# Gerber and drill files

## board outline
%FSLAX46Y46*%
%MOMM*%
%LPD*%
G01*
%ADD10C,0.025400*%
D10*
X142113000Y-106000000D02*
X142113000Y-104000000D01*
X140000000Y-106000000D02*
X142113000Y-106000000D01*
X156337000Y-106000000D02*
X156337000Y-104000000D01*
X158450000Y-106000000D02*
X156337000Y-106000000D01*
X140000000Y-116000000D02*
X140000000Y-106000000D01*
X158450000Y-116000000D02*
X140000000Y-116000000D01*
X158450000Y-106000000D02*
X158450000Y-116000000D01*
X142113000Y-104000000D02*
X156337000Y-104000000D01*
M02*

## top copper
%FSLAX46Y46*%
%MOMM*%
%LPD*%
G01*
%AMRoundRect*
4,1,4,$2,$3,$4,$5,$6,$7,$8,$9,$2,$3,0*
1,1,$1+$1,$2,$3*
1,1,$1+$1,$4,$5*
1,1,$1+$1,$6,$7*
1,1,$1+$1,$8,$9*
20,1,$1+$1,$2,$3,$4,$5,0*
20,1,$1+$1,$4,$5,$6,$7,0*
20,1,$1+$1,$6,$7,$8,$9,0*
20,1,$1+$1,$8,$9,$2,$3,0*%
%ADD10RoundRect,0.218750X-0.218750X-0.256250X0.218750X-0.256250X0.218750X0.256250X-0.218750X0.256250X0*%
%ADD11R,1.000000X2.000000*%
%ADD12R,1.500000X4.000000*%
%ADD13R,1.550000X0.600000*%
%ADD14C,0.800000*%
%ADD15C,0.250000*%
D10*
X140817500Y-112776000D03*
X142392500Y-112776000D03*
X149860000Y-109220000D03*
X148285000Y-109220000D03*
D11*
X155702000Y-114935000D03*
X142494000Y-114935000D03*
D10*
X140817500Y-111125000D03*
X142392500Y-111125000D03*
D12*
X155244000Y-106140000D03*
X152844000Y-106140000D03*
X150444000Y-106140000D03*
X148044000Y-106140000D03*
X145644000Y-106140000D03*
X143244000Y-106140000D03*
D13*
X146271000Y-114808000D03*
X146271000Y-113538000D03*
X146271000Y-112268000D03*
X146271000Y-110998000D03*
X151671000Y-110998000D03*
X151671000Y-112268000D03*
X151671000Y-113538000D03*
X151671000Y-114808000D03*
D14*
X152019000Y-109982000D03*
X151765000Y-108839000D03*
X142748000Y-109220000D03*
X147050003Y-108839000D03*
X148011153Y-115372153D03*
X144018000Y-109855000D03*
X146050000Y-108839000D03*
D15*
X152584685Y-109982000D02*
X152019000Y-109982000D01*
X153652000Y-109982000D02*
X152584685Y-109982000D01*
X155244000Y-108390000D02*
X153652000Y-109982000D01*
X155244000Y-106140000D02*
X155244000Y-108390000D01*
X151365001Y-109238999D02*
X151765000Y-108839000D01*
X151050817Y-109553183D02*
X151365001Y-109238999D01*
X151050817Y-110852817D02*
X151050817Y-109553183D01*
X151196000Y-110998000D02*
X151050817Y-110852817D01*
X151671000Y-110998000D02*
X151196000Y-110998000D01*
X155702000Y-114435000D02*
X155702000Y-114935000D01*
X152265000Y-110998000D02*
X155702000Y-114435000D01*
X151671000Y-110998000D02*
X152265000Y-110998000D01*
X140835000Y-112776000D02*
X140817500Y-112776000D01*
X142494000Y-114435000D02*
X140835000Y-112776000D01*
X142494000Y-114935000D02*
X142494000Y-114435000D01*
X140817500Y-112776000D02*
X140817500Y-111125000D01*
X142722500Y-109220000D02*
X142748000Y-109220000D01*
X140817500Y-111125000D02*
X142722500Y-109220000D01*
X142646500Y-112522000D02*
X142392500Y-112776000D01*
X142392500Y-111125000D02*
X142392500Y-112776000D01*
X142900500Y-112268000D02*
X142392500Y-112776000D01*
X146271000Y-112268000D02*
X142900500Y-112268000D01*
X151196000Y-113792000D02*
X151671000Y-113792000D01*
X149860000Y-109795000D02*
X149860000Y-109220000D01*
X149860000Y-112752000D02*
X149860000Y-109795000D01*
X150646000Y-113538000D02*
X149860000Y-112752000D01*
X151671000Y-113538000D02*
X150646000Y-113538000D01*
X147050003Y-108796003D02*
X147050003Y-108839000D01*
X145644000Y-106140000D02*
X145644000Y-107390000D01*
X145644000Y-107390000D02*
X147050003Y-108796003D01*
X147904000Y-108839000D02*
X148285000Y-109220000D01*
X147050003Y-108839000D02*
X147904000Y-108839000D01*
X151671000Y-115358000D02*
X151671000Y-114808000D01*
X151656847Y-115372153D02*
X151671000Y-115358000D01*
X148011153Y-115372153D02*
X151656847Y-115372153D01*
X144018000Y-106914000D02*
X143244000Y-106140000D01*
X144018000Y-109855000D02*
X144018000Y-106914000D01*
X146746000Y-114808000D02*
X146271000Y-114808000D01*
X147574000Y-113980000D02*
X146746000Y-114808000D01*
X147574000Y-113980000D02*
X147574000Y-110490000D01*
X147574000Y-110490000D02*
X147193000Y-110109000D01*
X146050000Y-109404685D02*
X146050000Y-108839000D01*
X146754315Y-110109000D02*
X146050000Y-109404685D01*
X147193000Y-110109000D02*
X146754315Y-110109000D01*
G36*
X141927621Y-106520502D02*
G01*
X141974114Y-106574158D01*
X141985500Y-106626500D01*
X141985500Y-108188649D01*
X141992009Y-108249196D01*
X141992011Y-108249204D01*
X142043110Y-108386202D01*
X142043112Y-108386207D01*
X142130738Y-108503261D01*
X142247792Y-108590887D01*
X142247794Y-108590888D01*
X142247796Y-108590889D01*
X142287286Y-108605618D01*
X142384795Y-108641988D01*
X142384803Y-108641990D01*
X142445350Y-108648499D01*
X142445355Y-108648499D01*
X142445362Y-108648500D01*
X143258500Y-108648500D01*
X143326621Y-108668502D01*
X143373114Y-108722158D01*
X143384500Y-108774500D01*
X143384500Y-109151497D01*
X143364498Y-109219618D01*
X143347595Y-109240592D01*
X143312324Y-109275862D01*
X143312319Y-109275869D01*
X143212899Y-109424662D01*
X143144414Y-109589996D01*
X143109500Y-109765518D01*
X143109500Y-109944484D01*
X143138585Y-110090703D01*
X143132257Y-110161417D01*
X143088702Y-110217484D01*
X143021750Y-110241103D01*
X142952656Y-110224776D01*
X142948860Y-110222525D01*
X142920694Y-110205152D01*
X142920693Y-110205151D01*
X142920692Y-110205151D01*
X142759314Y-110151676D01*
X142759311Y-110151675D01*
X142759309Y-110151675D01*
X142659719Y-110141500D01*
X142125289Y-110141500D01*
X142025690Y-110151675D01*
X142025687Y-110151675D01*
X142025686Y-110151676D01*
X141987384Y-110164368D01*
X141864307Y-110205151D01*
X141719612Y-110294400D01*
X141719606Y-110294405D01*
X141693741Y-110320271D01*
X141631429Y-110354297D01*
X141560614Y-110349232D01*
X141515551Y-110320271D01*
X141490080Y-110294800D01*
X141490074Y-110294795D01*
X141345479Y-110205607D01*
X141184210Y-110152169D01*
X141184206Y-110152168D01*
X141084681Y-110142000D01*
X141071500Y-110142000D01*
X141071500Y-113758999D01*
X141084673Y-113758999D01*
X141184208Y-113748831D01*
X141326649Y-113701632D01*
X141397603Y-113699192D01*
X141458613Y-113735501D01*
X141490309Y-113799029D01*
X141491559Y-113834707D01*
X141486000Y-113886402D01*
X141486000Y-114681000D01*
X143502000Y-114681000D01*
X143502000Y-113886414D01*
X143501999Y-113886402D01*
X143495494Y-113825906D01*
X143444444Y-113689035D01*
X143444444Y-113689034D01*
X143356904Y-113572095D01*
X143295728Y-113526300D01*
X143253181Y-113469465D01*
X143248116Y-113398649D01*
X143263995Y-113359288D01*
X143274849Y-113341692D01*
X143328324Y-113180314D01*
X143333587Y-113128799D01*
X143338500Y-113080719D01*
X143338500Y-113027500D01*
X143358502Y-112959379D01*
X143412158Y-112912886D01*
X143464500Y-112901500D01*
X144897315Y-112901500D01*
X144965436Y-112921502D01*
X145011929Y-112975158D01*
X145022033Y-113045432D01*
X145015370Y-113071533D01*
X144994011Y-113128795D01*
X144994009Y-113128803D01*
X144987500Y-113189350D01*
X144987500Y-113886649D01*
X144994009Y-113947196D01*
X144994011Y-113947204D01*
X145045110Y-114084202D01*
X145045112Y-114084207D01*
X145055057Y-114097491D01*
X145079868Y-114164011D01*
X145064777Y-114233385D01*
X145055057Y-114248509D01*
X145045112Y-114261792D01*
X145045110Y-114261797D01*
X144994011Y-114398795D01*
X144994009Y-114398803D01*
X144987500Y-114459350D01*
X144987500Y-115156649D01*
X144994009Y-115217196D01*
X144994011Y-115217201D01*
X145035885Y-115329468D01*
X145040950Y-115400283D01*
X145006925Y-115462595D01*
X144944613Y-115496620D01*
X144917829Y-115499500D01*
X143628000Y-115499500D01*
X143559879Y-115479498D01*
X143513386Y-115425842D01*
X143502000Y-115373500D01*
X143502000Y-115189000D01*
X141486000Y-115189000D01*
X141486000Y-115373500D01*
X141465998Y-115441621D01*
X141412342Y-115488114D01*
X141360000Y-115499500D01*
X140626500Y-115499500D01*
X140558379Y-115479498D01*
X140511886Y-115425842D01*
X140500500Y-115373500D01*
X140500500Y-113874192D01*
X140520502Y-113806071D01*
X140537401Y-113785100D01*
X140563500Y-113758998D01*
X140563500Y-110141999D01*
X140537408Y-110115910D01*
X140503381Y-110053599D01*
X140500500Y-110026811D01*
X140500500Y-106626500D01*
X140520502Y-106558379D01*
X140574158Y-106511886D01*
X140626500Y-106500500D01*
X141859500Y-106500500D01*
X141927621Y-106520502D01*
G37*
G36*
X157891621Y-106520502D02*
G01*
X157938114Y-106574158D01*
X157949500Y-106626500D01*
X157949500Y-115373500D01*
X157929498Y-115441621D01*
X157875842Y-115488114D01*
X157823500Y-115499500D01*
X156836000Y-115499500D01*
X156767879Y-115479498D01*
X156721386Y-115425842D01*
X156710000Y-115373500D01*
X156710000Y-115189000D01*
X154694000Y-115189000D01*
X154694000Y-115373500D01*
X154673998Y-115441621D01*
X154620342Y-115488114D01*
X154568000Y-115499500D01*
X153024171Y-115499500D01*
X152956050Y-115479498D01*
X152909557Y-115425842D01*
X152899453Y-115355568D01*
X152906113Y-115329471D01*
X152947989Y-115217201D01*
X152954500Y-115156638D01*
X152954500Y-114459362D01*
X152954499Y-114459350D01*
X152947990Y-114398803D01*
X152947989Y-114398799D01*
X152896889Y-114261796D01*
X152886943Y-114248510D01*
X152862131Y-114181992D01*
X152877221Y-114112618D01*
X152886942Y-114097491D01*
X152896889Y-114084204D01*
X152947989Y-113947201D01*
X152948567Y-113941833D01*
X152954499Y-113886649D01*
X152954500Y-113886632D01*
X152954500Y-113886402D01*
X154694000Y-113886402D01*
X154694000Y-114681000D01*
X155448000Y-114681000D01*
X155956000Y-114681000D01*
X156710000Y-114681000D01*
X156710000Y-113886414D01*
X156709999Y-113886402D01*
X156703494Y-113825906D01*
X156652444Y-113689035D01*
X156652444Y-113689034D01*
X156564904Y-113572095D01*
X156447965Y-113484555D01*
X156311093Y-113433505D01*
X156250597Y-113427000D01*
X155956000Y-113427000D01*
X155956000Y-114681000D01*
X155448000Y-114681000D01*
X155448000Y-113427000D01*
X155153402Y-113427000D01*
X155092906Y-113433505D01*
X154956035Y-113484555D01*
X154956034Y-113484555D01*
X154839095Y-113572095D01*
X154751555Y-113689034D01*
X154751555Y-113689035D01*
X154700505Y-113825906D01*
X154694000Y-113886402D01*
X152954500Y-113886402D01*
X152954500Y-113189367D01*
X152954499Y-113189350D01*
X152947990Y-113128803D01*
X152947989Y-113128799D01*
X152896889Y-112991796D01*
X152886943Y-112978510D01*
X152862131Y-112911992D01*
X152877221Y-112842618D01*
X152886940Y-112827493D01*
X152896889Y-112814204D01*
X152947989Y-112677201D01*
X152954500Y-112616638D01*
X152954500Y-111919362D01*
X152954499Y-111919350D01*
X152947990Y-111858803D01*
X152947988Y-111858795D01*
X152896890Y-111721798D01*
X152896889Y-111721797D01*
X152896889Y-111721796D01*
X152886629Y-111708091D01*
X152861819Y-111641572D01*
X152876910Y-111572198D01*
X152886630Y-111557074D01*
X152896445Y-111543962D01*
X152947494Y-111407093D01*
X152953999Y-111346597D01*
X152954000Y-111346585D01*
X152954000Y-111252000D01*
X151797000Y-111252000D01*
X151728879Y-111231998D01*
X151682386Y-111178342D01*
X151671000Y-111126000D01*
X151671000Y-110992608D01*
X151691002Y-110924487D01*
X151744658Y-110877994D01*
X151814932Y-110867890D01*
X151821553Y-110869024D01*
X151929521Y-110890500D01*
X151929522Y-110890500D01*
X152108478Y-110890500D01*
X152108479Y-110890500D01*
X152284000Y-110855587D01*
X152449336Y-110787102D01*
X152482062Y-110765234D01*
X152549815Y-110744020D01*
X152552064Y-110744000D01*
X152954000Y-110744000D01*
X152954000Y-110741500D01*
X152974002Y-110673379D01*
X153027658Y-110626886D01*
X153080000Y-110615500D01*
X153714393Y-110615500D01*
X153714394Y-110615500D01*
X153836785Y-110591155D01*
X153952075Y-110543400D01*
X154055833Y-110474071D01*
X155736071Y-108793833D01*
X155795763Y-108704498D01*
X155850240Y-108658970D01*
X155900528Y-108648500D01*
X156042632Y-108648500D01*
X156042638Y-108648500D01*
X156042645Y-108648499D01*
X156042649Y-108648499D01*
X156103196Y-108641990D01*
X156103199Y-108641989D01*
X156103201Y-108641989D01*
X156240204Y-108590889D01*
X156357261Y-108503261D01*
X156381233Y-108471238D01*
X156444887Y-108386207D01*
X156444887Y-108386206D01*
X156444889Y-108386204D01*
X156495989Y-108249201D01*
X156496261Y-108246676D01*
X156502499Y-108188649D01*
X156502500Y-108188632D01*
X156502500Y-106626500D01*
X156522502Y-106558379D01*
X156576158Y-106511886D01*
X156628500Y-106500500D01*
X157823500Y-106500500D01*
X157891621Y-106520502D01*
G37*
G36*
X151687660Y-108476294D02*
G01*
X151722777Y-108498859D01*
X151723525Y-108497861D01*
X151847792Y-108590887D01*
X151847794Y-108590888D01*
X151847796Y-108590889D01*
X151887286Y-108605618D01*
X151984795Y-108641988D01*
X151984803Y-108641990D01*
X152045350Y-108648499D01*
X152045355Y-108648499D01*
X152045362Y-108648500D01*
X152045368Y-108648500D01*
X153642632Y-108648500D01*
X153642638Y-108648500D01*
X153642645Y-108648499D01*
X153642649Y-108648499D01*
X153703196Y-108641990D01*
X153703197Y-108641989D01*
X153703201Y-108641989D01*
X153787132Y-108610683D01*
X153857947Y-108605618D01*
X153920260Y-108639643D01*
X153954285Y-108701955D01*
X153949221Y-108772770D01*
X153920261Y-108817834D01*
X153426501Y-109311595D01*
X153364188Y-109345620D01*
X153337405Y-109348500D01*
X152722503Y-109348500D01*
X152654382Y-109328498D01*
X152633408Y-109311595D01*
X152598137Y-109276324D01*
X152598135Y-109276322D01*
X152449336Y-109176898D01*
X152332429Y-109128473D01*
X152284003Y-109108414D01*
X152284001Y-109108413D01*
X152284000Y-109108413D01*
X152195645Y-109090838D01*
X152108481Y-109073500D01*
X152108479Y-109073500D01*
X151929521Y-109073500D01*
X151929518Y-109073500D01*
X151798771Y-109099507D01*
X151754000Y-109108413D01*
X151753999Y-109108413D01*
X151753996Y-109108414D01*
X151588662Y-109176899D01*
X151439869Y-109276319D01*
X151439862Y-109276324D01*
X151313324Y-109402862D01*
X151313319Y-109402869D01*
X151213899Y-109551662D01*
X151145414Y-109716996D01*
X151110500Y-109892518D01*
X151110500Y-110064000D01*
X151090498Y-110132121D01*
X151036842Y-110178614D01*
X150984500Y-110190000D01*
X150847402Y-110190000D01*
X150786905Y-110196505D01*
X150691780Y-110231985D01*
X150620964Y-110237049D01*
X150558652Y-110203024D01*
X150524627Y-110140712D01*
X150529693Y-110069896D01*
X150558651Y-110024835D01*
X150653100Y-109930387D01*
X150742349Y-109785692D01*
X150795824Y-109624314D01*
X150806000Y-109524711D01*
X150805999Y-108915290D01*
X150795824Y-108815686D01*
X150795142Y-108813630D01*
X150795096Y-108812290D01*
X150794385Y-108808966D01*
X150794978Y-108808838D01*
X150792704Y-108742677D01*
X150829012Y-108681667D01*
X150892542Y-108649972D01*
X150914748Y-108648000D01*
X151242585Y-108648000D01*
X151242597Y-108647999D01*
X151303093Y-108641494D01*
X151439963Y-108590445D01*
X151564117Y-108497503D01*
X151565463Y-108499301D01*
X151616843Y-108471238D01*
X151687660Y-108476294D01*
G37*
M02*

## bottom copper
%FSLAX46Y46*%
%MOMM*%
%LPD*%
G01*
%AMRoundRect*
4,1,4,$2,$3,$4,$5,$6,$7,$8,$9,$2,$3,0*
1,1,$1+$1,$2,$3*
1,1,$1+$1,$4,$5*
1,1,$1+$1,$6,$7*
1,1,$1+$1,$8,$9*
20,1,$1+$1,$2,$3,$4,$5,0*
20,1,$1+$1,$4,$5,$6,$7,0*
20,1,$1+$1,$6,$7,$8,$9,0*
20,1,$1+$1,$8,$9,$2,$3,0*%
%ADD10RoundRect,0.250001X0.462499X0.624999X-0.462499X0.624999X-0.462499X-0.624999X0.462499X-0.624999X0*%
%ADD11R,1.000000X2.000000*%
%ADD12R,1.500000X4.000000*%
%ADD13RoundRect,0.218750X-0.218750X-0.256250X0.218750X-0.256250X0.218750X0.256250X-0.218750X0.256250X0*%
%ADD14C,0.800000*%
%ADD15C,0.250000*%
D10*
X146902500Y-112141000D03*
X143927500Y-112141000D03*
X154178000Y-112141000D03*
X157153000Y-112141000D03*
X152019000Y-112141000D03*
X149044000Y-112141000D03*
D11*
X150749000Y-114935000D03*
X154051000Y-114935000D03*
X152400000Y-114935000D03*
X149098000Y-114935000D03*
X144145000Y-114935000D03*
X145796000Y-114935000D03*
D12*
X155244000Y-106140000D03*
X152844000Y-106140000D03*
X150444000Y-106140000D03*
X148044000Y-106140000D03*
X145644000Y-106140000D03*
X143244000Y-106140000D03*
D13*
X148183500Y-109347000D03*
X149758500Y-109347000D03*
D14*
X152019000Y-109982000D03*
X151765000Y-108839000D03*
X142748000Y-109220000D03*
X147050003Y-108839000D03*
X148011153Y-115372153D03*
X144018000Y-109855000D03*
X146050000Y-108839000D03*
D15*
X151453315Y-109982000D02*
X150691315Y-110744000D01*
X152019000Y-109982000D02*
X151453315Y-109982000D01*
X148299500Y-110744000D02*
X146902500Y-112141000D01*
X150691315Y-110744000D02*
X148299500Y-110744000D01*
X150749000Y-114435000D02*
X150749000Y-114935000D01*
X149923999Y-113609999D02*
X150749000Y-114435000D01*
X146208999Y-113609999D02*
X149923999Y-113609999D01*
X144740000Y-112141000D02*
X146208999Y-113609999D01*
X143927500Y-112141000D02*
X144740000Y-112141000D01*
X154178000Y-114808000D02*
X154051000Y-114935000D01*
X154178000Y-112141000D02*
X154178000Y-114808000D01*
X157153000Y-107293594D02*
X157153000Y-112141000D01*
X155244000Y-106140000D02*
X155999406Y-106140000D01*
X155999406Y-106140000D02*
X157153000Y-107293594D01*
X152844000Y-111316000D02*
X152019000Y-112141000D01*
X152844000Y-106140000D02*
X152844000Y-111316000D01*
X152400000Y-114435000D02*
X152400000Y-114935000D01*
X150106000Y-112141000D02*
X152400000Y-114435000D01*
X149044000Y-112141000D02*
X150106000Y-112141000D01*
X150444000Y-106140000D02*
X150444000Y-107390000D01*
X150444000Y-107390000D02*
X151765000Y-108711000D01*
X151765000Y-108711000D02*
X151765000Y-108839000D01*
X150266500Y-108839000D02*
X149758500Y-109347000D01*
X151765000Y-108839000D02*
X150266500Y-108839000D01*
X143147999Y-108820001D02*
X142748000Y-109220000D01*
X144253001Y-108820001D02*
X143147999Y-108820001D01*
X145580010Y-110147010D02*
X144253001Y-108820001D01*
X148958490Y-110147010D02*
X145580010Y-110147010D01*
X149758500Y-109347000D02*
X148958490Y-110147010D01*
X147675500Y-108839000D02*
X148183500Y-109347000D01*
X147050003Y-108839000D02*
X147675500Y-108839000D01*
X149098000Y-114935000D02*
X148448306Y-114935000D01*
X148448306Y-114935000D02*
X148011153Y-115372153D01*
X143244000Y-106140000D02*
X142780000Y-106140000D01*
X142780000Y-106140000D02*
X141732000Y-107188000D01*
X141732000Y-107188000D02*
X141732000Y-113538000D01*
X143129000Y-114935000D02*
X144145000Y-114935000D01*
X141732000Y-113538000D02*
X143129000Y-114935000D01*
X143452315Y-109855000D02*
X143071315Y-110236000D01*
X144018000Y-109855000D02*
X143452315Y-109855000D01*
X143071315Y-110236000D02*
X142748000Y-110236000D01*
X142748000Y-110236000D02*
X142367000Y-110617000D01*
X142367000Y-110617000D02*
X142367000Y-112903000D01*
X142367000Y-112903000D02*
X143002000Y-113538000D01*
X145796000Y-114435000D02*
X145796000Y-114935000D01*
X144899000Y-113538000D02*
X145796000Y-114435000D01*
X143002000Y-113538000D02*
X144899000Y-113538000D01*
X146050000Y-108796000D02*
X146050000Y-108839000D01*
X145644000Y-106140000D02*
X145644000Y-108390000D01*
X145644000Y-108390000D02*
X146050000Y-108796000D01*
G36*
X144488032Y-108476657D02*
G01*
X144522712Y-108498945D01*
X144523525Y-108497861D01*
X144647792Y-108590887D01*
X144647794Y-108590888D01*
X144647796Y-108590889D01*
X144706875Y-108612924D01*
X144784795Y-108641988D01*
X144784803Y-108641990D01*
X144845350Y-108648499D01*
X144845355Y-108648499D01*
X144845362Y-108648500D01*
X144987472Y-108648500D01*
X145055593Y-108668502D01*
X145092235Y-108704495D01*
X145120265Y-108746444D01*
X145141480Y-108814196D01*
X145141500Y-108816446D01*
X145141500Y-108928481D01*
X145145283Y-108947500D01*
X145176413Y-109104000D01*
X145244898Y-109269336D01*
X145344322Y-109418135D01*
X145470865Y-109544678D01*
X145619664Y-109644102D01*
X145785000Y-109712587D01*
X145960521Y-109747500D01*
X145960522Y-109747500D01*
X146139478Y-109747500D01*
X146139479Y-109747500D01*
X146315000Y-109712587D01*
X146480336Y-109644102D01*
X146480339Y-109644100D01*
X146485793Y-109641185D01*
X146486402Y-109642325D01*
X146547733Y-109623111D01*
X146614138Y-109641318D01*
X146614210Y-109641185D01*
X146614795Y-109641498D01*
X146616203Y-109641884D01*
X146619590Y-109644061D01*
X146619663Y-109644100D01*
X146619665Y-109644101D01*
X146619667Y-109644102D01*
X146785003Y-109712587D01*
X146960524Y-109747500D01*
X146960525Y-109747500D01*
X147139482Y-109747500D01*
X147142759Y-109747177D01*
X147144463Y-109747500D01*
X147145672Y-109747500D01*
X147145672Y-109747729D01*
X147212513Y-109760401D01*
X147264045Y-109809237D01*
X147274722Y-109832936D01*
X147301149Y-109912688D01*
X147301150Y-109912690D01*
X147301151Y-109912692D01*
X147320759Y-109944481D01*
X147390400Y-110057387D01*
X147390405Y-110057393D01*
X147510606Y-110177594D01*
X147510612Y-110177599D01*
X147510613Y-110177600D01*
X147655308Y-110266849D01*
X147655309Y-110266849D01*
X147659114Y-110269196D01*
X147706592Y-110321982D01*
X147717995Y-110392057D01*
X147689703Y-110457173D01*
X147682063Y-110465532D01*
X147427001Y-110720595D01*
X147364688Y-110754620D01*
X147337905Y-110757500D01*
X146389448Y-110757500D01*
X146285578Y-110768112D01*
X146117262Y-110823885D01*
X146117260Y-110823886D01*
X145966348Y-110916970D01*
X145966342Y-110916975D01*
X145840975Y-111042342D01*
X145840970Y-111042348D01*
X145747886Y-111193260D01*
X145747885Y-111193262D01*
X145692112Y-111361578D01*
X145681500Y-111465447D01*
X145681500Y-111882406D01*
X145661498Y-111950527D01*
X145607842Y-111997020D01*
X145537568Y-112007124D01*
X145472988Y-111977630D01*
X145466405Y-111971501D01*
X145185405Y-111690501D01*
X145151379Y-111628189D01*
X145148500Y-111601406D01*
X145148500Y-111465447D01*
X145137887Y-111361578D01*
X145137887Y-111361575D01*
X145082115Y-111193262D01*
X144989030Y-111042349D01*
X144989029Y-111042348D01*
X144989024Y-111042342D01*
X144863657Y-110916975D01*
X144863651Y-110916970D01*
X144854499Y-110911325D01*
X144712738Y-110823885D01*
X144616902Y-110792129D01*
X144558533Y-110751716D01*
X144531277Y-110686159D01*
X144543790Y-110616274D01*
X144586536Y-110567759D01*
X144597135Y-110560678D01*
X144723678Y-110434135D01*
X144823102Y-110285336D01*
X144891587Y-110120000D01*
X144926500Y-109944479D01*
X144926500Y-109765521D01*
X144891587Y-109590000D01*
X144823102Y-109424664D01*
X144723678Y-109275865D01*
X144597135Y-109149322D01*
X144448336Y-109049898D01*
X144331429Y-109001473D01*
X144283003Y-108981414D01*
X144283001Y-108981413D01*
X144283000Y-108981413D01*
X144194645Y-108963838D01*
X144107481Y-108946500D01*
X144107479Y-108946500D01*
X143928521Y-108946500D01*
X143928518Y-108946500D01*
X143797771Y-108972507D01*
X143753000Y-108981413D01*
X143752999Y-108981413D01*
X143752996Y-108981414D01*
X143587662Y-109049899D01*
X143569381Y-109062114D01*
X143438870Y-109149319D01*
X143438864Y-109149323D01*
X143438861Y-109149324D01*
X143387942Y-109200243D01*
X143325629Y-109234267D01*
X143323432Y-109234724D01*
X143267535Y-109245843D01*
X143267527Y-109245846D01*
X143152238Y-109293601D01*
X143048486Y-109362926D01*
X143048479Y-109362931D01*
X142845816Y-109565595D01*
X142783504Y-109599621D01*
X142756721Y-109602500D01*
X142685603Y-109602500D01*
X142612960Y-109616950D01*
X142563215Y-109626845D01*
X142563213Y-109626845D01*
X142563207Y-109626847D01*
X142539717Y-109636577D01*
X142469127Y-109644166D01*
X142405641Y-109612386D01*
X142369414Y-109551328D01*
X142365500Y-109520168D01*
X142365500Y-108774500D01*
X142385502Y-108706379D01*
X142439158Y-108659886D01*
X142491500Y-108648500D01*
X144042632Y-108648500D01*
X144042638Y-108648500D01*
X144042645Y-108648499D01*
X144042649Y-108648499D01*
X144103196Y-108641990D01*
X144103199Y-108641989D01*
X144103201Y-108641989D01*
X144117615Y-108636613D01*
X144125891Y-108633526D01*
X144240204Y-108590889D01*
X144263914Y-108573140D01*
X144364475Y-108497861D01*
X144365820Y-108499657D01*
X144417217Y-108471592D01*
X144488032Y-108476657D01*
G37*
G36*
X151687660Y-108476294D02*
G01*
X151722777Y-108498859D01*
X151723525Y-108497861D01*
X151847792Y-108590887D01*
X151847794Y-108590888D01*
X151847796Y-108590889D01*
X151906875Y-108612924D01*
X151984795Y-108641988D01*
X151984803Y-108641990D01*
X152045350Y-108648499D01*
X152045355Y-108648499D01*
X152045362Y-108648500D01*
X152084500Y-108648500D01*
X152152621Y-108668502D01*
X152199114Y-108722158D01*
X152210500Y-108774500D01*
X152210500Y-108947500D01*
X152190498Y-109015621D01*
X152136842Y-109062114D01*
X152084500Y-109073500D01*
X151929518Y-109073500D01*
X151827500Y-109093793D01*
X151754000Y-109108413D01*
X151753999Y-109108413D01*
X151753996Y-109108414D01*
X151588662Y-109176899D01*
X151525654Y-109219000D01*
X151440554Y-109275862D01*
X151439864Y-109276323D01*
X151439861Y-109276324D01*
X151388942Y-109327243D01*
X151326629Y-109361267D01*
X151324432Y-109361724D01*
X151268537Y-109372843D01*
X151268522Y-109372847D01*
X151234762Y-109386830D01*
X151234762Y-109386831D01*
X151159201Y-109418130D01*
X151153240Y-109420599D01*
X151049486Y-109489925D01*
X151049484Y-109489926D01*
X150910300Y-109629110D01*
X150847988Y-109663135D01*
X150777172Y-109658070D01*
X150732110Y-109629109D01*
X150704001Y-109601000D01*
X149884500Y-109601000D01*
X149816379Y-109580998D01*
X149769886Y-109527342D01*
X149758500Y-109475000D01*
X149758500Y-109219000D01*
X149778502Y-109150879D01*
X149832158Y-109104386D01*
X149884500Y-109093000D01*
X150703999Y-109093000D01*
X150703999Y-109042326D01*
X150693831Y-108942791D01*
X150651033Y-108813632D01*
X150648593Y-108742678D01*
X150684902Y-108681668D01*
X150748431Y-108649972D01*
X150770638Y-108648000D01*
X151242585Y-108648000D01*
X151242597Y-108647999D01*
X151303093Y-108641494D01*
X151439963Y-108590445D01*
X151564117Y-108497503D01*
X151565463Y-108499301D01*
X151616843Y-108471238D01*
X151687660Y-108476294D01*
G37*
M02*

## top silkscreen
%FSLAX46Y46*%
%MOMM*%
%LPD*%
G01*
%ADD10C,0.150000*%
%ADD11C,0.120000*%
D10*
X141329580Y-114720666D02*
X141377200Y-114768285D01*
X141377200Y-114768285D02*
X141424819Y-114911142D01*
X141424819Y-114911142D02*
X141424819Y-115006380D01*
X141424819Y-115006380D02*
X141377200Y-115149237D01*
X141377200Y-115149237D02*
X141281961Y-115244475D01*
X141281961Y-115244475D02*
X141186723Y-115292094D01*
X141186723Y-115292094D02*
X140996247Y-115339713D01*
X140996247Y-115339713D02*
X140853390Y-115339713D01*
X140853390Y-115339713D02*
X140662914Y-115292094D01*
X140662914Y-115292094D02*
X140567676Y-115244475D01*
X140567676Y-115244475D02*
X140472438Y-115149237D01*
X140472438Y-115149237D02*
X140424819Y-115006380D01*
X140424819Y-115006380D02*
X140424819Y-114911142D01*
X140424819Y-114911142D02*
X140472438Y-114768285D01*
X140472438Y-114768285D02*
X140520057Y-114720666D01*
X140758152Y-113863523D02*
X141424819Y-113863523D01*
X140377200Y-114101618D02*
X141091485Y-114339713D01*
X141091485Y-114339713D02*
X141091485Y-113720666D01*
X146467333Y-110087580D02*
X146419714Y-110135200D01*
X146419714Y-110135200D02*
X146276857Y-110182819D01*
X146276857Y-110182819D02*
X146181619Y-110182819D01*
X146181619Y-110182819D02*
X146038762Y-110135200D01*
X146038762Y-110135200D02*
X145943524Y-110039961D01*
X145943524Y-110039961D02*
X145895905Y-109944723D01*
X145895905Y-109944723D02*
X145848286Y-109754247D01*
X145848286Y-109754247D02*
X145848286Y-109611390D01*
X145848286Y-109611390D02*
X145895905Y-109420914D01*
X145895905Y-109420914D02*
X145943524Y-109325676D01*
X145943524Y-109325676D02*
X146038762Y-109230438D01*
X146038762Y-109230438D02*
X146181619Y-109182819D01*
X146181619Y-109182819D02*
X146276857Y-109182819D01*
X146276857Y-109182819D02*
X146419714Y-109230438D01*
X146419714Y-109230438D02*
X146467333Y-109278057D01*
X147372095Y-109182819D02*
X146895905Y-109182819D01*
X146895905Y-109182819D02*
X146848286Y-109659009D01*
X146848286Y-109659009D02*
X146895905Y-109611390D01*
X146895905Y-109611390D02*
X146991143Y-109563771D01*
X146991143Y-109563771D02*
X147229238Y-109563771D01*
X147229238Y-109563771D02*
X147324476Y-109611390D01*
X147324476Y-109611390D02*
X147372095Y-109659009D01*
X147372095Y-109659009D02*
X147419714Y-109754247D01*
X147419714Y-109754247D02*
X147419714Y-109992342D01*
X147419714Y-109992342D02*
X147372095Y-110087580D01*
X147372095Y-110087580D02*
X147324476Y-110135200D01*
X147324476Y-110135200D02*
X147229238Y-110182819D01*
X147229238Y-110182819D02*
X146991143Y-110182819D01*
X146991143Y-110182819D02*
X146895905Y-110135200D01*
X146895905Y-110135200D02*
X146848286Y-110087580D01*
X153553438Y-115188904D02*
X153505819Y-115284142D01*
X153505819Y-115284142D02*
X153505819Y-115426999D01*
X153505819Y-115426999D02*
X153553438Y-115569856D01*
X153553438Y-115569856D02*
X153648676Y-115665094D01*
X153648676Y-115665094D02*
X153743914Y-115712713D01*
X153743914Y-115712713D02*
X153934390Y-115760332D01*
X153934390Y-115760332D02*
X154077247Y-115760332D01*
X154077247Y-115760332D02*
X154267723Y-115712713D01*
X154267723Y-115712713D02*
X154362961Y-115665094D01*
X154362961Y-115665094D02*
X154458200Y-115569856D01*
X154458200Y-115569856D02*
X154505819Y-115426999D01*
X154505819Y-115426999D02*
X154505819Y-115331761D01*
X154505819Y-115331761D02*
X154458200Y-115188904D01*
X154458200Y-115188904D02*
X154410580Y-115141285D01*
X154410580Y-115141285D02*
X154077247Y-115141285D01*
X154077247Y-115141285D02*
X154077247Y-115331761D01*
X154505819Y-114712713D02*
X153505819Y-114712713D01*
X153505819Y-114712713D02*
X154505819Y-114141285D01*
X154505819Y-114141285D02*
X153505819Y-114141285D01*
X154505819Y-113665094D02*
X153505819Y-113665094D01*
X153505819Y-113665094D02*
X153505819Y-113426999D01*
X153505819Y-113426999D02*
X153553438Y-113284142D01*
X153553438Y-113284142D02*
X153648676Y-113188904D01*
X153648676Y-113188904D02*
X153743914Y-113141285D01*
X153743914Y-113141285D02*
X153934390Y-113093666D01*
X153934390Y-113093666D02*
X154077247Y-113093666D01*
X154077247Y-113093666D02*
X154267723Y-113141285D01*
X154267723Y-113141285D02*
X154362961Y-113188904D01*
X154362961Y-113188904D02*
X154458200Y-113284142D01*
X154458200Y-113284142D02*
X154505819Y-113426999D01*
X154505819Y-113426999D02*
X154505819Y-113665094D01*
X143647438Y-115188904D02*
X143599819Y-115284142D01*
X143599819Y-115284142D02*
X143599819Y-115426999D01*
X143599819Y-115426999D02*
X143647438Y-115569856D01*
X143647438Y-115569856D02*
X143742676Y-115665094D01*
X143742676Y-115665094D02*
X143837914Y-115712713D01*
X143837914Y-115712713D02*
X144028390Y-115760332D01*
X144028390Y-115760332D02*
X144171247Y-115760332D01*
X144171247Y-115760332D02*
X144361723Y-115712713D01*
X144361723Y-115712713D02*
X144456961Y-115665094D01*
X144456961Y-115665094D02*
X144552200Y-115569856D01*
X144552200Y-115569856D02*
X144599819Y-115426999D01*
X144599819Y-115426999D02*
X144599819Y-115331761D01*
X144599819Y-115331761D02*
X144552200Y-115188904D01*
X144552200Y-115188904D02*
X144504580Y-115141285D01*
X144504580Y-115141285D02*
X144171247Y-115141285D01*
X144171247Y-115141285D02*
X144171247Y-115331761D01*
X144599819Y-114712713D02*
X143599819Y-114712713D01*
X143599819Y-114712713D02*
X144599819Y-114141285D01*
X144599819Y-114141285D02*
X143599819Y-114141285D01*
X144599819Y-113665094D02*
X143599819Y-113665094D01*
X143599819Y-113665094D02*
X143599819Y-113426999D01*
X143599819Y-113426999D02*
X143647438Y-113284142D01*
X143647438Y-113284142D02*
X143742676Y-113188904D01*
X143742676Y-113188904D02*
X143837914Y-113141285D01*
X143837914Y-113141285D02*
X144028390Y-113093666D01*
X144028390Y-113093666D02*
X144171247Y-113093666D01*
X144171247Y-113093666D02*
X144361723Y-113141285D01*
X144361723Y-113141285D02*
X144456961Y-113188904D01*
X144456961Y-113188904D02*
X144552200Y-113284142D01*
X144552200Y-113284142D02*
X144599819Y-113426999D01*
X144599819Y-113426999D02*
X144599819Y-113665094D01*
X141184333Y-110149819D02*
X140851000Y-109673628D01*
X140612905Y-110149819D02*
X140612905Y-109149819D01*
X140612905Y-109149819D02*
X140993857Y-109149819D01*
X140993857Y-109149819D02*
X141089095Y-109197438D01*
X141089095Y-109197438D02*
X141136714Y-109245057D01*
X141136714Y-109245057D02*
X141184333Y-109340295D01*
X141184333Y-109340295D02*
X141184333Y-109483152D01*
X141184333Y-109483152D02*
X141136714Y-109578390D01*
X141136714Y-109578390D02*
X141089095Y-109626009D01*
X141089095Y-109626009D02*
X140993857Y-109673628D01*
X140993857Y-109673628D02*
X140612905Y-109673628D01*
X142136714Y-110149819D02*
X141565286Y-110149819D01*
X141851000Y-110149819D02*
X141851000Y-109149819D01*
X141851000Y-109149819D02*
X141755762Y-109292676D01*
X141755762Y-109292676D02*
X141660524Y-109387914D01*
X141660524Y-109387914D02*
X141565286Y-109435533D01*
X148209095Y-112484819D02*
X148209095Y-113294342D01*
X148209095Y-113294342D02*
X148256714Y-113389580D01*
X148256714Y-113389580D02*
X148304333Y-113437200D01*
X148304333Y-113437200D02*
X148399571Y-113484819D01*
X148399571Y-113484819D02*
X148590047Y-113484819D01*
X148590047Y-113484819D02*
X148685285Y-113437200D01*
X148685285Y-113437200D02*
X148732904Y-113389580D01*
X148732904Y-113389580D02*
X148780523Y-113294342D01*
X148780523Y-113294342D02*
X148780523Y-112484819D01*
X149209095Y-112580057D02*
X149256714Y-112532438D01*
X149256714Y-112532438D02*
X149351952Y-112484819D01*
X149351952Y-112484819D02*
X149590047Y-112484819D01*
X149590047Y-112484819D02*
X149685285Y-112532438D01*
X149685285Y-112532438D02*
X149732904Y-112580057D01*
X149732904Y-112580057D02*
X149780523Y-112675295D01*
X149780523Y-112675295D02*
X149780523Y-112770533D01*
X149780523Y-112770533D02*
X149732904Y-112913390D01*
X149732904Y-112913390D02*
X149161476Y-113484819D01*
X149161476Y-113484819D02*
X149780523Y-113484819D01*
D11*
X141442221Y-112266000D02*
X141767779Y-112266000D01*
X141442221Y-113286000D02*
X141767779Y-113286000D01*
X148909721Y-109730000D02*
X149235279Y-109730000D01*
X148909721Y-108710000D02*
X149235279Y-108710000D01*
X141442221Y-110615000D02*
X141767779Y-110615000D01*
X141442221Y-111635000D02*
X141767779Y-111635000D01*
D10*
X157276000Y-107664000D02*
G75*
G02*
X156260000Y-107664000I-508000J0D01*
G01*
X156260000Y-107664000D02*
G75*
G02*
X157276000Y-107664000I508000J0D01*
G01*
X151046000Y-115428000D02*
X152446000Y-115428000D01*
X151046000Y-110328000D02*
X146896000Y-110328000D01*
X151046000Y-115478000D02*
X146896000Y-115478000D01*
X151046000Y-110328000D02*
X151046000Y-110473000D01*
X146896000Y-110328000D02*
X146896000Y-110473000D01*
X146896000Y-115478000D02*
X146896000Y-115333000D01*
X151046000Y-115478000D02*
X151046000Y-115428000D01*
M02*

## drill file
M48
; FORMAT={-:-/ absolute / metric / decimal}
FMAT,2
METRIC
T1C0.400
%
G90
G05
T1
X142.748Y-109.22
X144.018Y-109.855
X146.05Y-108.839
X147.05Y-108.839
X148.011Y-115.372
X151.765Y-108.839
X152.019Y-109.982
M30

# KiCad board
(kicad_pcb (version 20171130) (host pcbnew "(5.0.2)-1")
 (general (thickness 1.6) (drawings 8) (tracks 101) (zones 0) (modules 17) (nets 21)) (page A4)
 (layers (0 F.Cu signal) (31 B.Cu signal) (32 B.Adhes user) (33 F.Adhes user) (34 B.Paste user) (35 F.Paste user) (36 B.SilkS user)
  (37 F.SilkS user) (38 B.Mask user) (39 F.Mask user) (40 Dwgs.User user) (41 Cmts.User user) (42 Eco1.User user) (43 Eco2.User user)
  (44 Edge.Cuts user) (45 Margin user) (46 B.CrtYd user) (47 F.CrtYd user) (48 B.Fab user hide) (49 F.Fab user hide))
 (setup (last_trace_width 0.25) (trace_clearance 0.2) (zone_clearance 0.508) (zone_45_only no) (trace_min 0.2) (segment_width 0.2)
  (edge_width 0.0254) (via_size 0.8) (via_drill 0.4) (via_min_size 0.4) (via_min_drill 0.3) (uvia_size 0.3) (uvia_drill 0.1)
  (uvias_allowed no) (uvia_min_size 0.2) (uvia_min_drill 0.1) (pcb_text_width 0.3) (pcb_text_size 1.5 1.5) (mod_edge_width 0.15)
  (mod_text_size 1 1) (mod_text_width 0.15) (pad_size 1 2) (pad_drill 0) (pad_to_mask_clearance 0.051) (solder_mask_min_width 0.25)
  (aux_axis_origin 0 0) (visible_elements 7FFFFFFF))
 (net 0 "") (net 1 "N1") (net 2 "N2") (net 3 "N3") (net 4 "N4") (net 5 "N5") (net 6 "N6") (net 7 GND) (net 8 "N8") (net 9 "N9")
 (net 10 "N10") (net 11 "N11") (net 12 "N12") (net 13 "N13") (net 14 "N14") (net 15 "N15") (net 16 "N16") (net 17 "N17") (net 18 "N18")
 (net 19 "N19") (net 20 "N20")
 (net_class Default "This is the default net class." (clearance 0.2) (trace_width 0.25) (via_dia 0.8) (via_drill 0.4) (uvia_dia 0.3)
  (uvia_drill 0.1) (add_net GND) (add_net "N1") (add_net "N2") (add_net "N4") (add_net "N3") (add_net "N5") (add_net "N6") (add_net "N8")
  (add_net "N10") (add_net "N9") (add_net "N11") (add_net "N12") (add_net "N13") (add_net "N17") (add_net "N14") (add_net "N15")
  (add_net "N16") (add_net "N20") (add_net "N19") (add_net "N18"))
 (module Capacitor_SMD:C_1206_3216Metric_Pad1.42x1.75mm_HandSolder (layer B.Cu) (at 145.415 112.141 180)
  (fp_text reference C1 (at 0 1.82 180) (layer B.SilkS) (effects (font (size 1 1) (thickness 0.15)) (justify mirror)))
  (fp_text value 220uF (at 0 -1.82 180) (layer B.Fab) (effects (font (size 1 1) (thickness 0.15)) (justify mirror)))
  (pad 1 smd roundrect (at -1.4875 0 180) (size 1.425 1.75) (layers B.Cu B.Paste B.Mask) (roundrect_rratio 0.175439) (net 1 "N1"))
  (pad 2 smd roundrect (at 1.4875 0 180) (size 1.425 1.75) (layers B.Cu B.Paste B.Mask) (roundrect_rratio 0.175439) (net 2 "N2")))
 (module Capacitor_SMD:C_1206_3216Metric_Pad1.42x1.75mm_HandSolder (layer B.Cu) (at 155.6655 112.141 180)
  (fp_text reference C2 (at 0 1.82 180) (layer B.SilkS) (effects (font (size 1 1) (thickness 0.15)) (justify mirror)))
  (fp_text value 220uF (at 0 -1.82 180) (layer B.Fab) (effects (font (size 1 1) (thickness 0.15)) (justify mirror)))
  (pad 2 smd roundrect (at 1.4875 0 180) (size 1.425 1.75) (layers B.Cu B.Paste B.Mask) (roundrect_rratio 0.175439) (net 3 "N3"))
  (pad 1 smd roundrect (at -1.4875 0 180) (size 1.425 1.75) (layers B.Cu B.Paste B.Mask) (roundrect_rratio 0.175439) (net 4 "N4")))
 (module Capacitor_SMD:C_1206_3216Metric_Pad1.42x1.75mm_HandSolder (layer B.Cu) (at 150.5315 112.141 180)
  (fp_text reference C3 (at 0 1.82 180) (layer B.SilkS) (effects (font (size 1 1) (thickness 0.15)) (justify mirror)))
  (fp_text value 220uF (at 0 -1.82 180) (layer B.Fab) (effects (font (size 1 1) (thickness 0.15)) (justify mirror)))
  (pad 1 smd roundrect (at -1.4875 0 180) (size 1.425 1.75) (layers B.Cu B.Paste B.Mask) (roundrect_rratio 0.175439) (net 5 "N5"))
  (pad 2 smd roundrect (at 1.4875 0 180) (size 1.425 1.75) (layers B.Cu B.Paste B.Mask) (roundrect_rratio 0.175439) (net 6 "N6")))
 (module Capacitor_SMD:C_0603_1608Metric (layer F.Cu) (at 141.605 112.776)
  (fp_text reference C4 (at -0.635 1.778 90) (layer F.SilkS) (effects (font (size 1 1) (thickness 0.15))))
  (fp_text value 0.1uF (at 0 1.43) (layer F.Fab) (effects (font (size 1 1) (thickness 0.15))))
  (fp_line (start -0.162779 -0.51) (end 0.162779 -0.51) (layer F.SilkS) (width 0.12))
  (fp_line (start -0.162779 0.51) (end 0.162779 0.51) (layer F.SilkS) (width 0.12))
  (pad 1 smd roundrect (at -0.7875 0) (size 0.875 0.95) (layers F.Cu F.Paste F.Mask) (roundrect_rratio 0.25) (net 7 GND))
  (pad 2 smd roundrect (at 0.7875 0) (size 0.875 0.95) (layers F.Cu F.Paste F.Mask) (roundrect_rratio 0.25) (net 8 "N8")))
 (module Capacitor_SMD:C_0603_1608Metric (layer F.Cu) (at 149.0725 109.22)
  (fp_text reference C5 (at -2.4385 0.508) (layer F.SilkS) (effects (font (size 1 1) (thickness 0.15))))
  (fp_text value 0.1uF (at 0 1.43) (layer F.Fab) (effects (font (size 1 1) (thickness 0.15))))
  (fp_line (start -0.162779 0.51) (end 0.162779 0.51) (layer F.SilkS) (width 0.12))
  (fp_line (start -0.162779 -0.51) (end 0.162779 -0.51) (layer F.SilkS) (width 0.12))
  (pad 2 smd roundrect (at 0.7875 0) (size 0.875 0.95) (layers F.Cu F.Paste F.Mask) (roundrect_rratio 0.25) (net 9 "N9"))
  (pad 1 smd roundrect (at -0.7875 0) (size 0.875 0.95) (layers F.Cu F.Paste F.Mask) (roundrect_rratio 0.25) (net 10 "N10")))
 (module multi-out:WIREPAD (layer B.Cu) (at 150.749 114.935)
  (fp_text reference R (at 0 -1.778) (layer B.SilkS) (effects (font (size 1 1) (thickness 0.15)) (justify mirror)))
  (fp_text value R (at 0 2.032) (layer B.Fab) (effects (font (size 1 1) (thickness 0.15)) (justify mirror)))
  (pad 1 connect rect (at 0 0) (size 1 2) (layers B.Cu B.Mask) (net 2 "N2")))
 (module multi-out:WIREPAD (layer B.Cu) (at 154.051 114.935)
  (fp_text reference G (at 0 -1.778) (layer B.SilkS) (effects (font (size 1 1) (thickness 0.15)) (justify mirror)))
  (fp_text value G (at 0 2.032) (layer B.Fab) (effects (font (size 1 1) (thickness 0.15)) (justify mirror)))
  (pad 1 connect rect (at 0 0) (size 1 2) (layers B.Cu B.Mask) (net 3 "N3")))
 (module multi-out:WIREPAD (layer B.Cu) (at 152.4 114.935)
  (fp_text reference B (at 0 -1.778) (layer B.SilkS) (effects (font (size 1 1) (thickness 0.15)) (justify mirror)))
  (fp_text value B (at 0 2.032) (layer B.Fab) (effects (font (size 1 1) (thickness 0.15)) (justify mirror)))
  (pad 1 connect rect (at 0 0) (size 1 2) (layers B.Cu B.Mask) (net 6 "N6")))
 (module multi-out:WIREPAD (layer B.Cu) (at 149.098 114.935)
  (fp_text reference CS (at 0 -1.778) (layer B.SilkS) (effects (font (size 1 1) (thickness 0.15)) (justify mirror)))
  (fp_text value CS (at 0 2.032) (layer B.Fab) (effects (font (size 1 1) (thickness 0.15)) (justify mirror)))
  (pad 1 connect rect (at 0 0) (size 1 2) (layers B.Cu B.Mask) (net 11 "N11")))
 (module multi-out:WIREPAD (layer F.Cu) (at 155.702 114.935)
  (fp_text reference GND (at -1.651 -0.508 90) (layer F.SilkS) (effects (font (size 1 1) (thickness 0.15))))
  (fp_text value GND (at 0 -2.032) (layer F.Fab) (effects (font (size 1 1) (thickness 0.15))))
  (pad 1 connect rect (at 0 0) (size 1 2) (layers F.Cu F.Mask) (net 7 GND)))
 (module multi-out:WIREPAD (layer B.Cu) (at 144.145 114.935)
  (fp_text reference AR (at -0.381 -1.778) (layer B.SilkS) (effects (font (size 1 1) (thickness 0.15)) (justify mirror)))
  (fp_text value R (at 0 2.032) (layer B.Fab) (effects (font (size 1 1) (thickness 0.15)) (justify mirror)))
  (pad 1 connect rect (at 0 0) (size 1 2) (layers B.Cu B.Mask) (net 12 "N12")))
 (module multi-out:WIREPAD (layer B.Cu) (at 145.796 114.935)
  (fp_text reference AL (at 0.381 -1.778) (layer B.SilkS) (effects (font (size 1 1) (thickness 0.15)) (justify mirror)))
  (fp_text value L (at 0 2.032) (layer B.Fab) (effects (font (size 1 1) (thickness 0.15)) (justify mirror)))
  (pad 1 connect rect (at 0 0) (size 1 2) (layers B.Cu B.Mask) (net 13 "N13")))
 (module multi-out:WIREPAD (layer F.Cu) (at 142.494 114.935)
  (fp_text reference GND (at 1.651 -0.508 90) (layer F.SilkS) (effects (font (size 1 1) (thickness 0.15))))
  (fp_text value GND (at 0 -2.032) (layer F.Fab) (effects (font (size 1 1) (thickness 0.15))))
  (pad 1 connect rect (at 0 0) (size 1 2) (layers F.Cu F.Mask) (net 7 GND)))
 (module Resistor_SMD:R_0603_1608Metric (layer F.Cu) (at 141.605 111.125)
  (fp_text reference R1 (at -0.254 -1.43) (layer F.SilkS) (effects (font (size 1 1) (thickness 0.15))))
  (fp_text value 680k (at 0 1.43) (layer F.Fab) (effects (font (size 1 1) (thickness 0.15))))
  (fp_line (start -0.162779 -0.51) (end 0.162779 -0.51) (layer F.SilkS) (width 0.12))
  (fp_line (start -0.162779 0.51) (end 0.162779 0.51) (layer F.SilkS) (width 0.12))
  (pad 1 smd roundrect (at -0.7875 0) (size 0.875 0.95) (layers F.Cu F.Paste F.Mask) (roundrect_rratio 0.25) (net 7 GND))
  (pad 2 smd roundrect (at 0.7875 0) (size 0.875 0.95) (layers F.Cu F.Paste F.Mask) (roundrect_rratio 0.25) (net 8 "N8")))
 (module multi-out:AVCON (layer F.Cu) (at 149.148 106.14)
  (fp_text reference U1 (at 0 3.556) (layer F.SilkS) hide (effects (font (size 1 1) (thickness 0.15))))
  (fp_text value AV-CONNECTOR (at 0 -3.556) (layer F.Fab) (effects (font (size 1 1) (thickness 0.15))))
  (fp_circle (center 7.62 1.524) (end 8.128 1.524) (layer F.SilkS) (width 0.15))
  (pad 1 connect rect (at 6.096 0) (size 1.5 4) (layers F.Cu F.Mask) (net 1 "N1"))
  (pad 3 connect rect (at 3.696 0) (size 1.5 4) (layers F.Cu F.Mask) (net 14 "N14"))
  (pad 5 connect rect (at 1.296 0) (size 1.5 4) (layers F.Cu F.Mask) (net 7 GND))
  (pad 7 connect rect (at -1.104 0) (size 1.5 4) (layers F.Cu F.Mask) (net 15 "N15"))
  (pad 9 connect rect (at -3.504 0) (size 1.5 4) (layers F.Cu F.Mask) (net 10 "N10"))
  (pad 11 connect rect (at -5.904 0) (size 1.5 4) (layers F.Cu F.Mask) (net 13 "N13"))
  (pad 2 connect rect (at 6.096 0) (size 1.5 4) (layers B.Cu B.Mask) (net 4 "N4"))
  (pad 4 connect rect (at 3.696 0) (size 1.5 4) (layers B.Cu B.Mask) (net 5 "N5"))
  (pad 6 connect rect (at 1.296 0) (size 1.5 4) (layers B.Cu B.Mask) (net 7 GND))
  (pad 8 connect rect (at -1.104 0) (size 1.5 4) (layers B.Cu B.Mask) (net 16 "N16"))
  (pad 10 connect rect (at -3.504 0) (size 1.5 4) (layers B.Cu B.Mask) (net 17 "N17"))
  (pad 12 connect rect (at -5.904 0) (size 1.5 4) (layers B.Cu B.Mask) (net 12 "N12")))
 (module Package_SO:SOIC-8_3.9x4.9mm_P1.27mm (layer F.Cu) (at 148.971 112.903 180)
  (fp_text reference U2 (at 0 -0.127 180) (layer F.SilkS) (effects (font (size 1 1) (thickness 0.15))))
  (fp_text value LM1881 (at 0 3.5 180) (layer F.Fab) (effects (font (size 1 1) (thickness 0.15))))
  (fp_line (start -2.075 -2.525) (end -3.475 -2.525) (layer F.SilkS) (width 0.15))
  (fp_line (start -2.075 2.575) (end 2.075 2.575) (layer F.SilkS) (width 0.15))
  (fp_line (start -2.075 -2.575) (end 2.075 -2.575) (layer F.SilkS) (width 0.15))
  (fp_line (start -2.075 2.575) (end -2.075 2.43) (layer F.SilkS) (width 0.15))
  (fp_line (start 2.075 2.575) (end 2.075 2.43) (layer F.SilkS) (width 0.15))
  (fp_line (start 2.075 -2.575) (end 2.075 -2.43) (layer F.SilkS) (width 0.15))
  (fp_line (start -2.075 -2.575) (end -2.075 -2.525) (layer F.SilkS) (width 0.15))
  (pad 8 smd rect (at 2.7 -1.905 180) (size 1.55 0.6) (layers F.Cu F.Paste F.Mask) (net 17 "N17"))
  (pad 7 smd rect (at 2.7 -0.635 180) (size 1.55 0.6) (layers F.Cu F.Paste F.Mask) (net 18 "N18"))
  (pad 6 smd rect (at 2.7 0.635 180) (size 1.55 0.6) (layers F.Cu F.Paste F.Mask) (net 8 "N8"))
  (pad 5 smd rect (at 2.7 1.905 180) (size 1.55 0.6) (layers F.Cu F.Paste F.Mask) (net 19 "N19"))
  (pad 4 smd rect (at -2.7 1.905 180) (size 1.55 0.6) (layers F.Cu F.Paste F.Mask) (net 7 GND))
  (pad 3 smd rect (at -2.7 0.635 180) (size 1.55 0.6) (layers F.Cu F.Paste F.Mask) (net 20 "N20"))
  (pad 2 smd rect (at -2.7 -0.635 180) (size 1.55 0.6) (layers F.Cu F.Paste F.Mask) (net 9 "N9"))
  (pad 1 smd rect (at -2.7 -1.905 180) (size 1.55 0.6) (layers F.Cu F.Paste F.Mask) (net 11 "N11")))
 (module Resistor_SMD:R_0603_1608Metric (layer B.Cu) (at 148.971 109.347)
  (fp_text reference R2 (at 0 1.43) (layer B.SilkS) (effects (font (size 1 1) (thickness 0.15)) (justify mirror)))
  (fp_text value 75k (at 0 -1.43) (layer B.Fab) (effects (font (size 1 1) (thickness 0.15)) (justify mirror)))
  (pad 1 smd roundrect (at -0.7875 0) (size 0.875 0.95) (layers B.Cu B.Paste B.Mask) (roundrect_rratio 0.25) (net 10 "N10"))
  (pad 2 smd roundrect (at 0.7875 0) (size 0.875 0.95) (layers B.Cu B.Paste B.Mask) (roundrect_rratio 0.25) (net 7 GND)))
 (gr_line (start 142.113 106) (end 142.113 104) (layer Edge.Cuts) (width 0.0254))
 (gr_line (start 140 106) (end 142.113 106) (layer Edge.Cuts) (width 0.0254))
 (gr_line (start 156.337 106) (end 156.337 104) (layer Edge.Cuts) (width 0.0254))
 (gr_line (start 158.45 106) (end 156.337 106) (layer Edge.Cuts) (width 0.0254))
 (gr_line (start 140 116) (end 140 106) (layer Edge.Cuts) (width 0.0254))
 (gr_line (start 158.45 116) (end 140 116) (layer Edge.Cuts) (width 0.0254))
 (gr_line (start 158.45 106) (end 158.45 116) (layer Edge.Cuts) (width 0.0254))
 (gr_line (start 142.113 104) (end 156.337 104) (layer Edge.Cuts) (width 0.0254))
 (via (at 152.019 109.982) (size 0.8) (drill 0.4) (layers F.Cu B.Cu) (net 1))
 (segment (start 152.584685 109.982) (end 152.019 109.982) (width 0.25) (layer F.Cu) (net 1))
 (segment (start 153.652 109.982) (end 152.584685 109.982) (width 0.25) (layer F.Cu) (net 1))
 (segment (start 155.244 108.39) (end 153.652 109.982) (width 0.25) (layer F.Cu) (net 1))
 (segment (start 155.244 106.14) (end 155.244 108.39) (width 0.25) (layer F.Cu) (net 1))
 (segment (start 151.453315 109.982) (end 150.691315 110.744) (width 0.25) (layer B.Cu) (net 1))
 (segment (start 152.019 109.982) (end 151.453315 109.982) (width 0.25) (layer B.Cu) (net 1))
 (segment (start 148.2995 110.744) (end 146.9025 112.141) (width 0.25) (layer B.Cu) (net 1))
 (segment (start 150.691315 110.744) (end 148.2995 110.744) (width 0.25) (layer B.Cu) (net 1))
 (segment (start 150.749 114.435) (end 150.749 114.935) (width 0.25) (layer B.Cu) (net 2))
 (segment (start 149.923999 113.609999) (end 150.749 114.435) (width 0.25) (layer B.Cu) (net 2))
 (segment (start 146.208999 113.609999) (end 149.923999 113.609999) (width 0.25) (layer B.Cu) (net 2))
 (segment (start 144.74 112.141) (end 146.208999 113.609999) (width 0.25) (layer B.Cu) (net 2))
 (segment (start 143.9275 112.141) (end 144.74 112.141) (width 0.25) (layer B.Cu) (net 2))
 (segment (start 154.178 114.808) (end 154.051 114.935) (width 0.25) (layer B.Cu) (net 3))
 (segment (start 154.178 112.141) (end 154.178 114.808) (width 0.25) (layer B.Cu) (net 3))
 (segment (start 157.153 107.293594) (end 157.153 112.141) (width 0.25) (layer B.Cu) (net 4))
 (segment (start 155.244 106.14) (end 155.999406 106.14) (width 0.25) (layer B.Cu) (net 4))
 (segment (start 155.999406 106.14) (end 157.153 107.293594) (width 0.25) (layer B.Cu) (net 4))
 (segment (start 152.844 111.316) (end 152.019 112.141) (width 0.25) (layer B.Cu) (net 5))
 (segment (start 152.844 106.14) (end 152.844 111.316) (width 0.25) (layer B.Cu) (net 5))
 (segment (start 152.4 114.435) (end 152.4 114.935) (width 0.25) (layer B.Cu) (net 6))
 (segment (start 150.106 112.141) (end 152.4 114.435) (width 0.25) (layer B.Cu) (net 6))
 (segment (start 149.044 112.141) (end 150.106 112.141) (width 0.25) (layer B.Cu) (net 6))
 (via (at 151.765 108.839) (size 0.8) (drill 0.4) (layers F.Cu B.Cu) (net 7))
 (via (at 142.748 109.22) (size 0.8) (drill 0.4) (layers F.Cu B.Cu) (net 7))
 (segment (start 151.365001 109.238999) (end 151.765 108.839) (width 0.25) (layer F.Cu) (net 7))
 (segment (start 151.050817 109.553183) (end 151.365001 109.238999) (width 0.25) (layer F.Cu) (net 7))
 (segment (start 151.050817 110.852817) (end 151.050817 109.553183) (width 0.25) (layer F.Cu) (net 7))
 (segment (start 151.196 110.998) (end 151.050817 110.852817) (width 0.25) (layer F.Cu) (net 7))
 (segment (start 151.671 110.998) (end 151.196 110.998) (width 0.25) (layer F.Cu) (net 7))
 (segment (start 150.444 106.14) (end 150.444 107.39) (width 0.25) (layer B.Cu) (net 7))
 (segment (start 150.444 107.39) (end 151.765 108.711) (width 0.25) (layer B.Cu) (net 7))
 (segment (start 151.765 108.711) (end 151.765 108.839) (width 0.25) (layer B.Cu) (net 7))
 (segment (start 150.2665 108.839) (end 149.7585 109.347) (width 0.25) (layer B.Cu) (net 7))
 (segment (start 151.765 108.839) (end 150.2665 108.839) (width 0.25) (layer B.Cu) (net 7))
 (segment (start 143.147999 108.820001) (end 142.748 109.22) (width 0.25) (layer B.Cu) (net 7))
 (segment (start 144.253001 108.820001) (end 143.147999 108.820001) (width 0.25) (layer B.Cu) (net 7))
 (segment (start 145.58001 110.14701) (end 144.253001 108.820001) (width 0.25) (layer B.Cu) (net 7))
 (segment (start 148.95849 110.14701) (end 145.58001 110.14701) (width 0.25) (layer B.Cu) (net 7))
 (segment (start 149.7585 109.347) (end 148.95849 110.14701) (width 0.25) (layer B.Cu) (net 7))
 (segment (start 155.702 114.435) (end 155.702 114.935) (width 0.25) (layer F.Cu) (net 7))
 (segment (start 152.265 110.998) (end 155.702 114.435) (width 0.25) (layer F.Cu) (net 7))
 (segment (start 151.671 110.998) (end 152.265 110.998) (width 0.25) (layer F.Cu) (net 7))
 (segment (start 140.835 112.776) (end 140.8175 112.776) (width 0.25) (layer F.Cu) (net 7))
 (segment (start 142.494 114.435) (end 140.835 112.776) (width 0.25) (layer F.Cu) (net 7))
 (segment (start 142.494 114.935) (end 142.494 114.435) (width 0.25) (layer F.Cu) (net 7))
 (segment (start 140.8175 112.776) (end 140.8175 111.125) (width 0.25) (layer F.Cu) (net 7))
 (segment (start 142.7225 109.22) (end 142.748 109.22) (width 0.25) (layer F.Cu) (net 7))
 (segment (start 140.8175 111.125) (end 142.7225 109.22) (width 0.25) (layer F.Cu) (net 7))
 (segment (start 142.6465 112.522) (end 142.3925 112.776) (width 0.25) (layer F.Cu) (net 8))
 (segment (start 142.3925 111.125) (end 142.3925 112.776) (width 0.25) (layer F.Cu) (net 8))
 (segment (start 142.9005 112.268) (end 142.3925 112.776) (width 0.25) (layer F.Cu) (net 8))
 (segment (start 146.271 112.268) (end 142.9005 112.268) (width 0.25) (layer F.Cu) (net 8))
 (segment (start 151.196 113.792) (end 151.671 113.792) (width 0.25) (layer F.Cu) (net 9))
 (segment (start 149.86 109.795) (end 149.86 109.22) (width 0.25) (layer F.Cu) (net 9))
 (segment (start 149.86 112.752) (end 149.86 109.795) (width 0.25) (layer F.Cu) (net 9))
 (segment (start 150.646 113.538) (end 149.86 112.752) (width 0.25) (layer F.Cu) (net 9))
 (segment (start 151.671 113.538) (end 150.646 113.538) (width 0.25) (layer F.Cu) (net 9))
 (via (at 147.050003 108.839) (size 0.8) (drill 0.4) (layers F.Cu B.Cu) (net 10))
 (segment (start 147.050003 108.796003) (end 147.050003 108.839) (width 0.25) (layer F.Cu) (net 10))
 (segment (start 145.644 106.14) (end 145.644 107.39) (width 0.25) (layer F.Cu) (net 10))
 (segment (start 145.644 107.39) (end 147.050003 108.796003) (width 0.25) (layer F.Cu) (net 10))
 (segment (start 147.6755 108.839) (end 148.1835 109.347) (width 0.25) (layer B.Cu) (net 10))
 (segment (start 147.050003 108.839) (end 147.6755 108.839) (width 0.25) (layer B.Cu) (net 10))
 (segment (start 147.904 108.839) (end 148.285 109.22) (width 0.25) (layer F.Cu) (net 10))
 (segment (start 147.050003 108.839) (end 147.904 108.839) (width 0.25) (layer F.Cu) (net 10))
 (via (at 148.011153 115.372153) (size 0.8) (drill 0.4) (layers F.Cu B.Cu) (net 11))
 (segment (start 149.098 114.935) (end 148.448306 114.935) (width 0.25) (layer B.Cu) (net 11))
 (segment (start 148.448306 114.935) (end 148.011153 115.372153) (width 0.25) (layer B.Cu) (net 11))
 (segment (start 151.671 115.358) (end 151.671 114.808) (width 0.25) (layer F.Cu) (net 11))
 (segment (start 151.656847 115.372153) (end 151.671 115.358) (width 0.25) (layer F.Cu) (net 11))
 (segment (start 148.011153 115.372153) (end 151.656847 115.372153) (width 0.25) (layer F.Cu) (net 11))
 (segment (start 143.244 106.14) (end 142.78 106.14) (width 0.25) (layer B.Cu) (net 12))
 (segment (start 142.78 106.14) (end 141.732 107.188) (width 0.25) (layer B.Cu) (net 12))
 (segment (start 141.732 107.188) (end 141.732 113.538) (width 0.25) (layer B.Cu) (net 12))
 (segment (start 143.129 114.935) (end 144.145 114.935) (width 0.25) (layer B.Cu) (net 12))
 (segment (start 141.732 113.538) (end 143.129 114.935) (width 0.25) (layer B.Cu) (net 12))
 (via (at 144.018 109.855) (size 0.8) (drill 0.4) (layers F.Cu B.Cu) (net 13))
 (segment (start 144.018 106.914) (end 143.244 106.14) (width 0.25) (layer F.Cu) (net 13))
 (segment (start 144.018 109.855) (end 144.018 106.914) (width 0.25) (layer F.Cu) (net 13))
 (segment (start 143.452315 109.855) (end 143.071315 110.236) (width 0.25) (layer B.Cu) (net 13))
 (segment (start 144.018 109.855) (end 143.452315 109.855) (width 0.25) (layer B.Cu) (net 13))
 (segment (start 143.071315 110.236) (end 142.748 110.236) (width 0.25) (layer B.Cu) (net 13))
 (segment (start 142.748 110.236) (end 142.367 110.617) (width 0.25) (layer B.Cu) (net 13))
 (segment (start 142.367 110.617) (end 142.367 112.903) (width 0.25) (layer B.Cu) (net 13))
 (segment (start 142.367 112.903) (end 143.002 113.538) (width 0.25) (layer B.Cu) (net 13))
 (segment (start 145.796 114.435) (end 145.796 114.935) (width 0.25) (layer B.Cu) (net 13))
 (segment (start 144.899 113.538) (end 145.796 114.435) (width 0.25) (layer B.Cu) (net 13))
 (segment (start 143.002 113.538) (end 144.899 113.538) (width 0.25) (layer B.Cu) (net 13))
 (via (at 146.05 108.839) (size 0.8) (drill 0.4) (layers F.Cu B.Cu) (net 17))
 (segment (start 146.05 108.796) (end 146.05 108.839) (width 0.25) (layer B.Cu) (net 17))
 (segment (start 145.644 106.14) (end 145.644 108.39) (width 0.25) (layer B.Cu) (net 17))
 (segment (start 145.644 108.39) (end 146.05 108.796) (width 0.25) (layer B.Cu) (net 17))
 (segment (start 146.746 114.808) (end 146.271 114.808) (width 0.25) (layer F.Cu) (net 17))
 (segment (start 147.574 113.98) (end 146.746 114.808) (width 0.25) (layer F.Cu) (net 17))
 (segment (start 147.574 113.98) (end 147.574 110.49) (width 0.25) (layer F.Cu) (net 17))
 (segment (start 147.574 110.49) (end 147.193 110.109) (width 0.25) (layer F.Cu) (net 17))
 (segment (start 146.05 109.404685) (end 146.05 108.839) (width 0.25) (layer F.Cu) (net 17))
 (segment (start 146.754315 110.109) (end 146.05 109.404685) (width 0.25) (layer F.Cu) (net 17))
 (segment (start 147.193 110.109) (end 146.754315 110.109) (width 0.25) (layer F.Cu) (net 17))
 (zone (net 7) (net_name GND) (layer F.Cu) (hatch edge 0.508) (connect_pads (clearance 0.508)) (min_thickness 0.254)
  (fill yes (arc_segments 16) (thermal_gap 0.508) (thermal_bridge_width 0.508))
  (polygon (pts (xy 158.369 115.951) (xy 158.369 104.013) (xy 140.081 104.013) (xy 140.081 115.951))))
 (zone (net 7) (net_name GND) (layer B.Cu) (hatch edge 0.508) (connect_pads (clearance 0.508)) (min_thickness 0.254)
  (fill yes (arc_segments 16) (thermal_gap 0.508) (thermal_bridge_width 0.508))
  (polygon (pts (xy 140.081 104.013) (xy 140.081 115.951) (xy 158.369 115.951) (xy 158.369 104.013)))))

